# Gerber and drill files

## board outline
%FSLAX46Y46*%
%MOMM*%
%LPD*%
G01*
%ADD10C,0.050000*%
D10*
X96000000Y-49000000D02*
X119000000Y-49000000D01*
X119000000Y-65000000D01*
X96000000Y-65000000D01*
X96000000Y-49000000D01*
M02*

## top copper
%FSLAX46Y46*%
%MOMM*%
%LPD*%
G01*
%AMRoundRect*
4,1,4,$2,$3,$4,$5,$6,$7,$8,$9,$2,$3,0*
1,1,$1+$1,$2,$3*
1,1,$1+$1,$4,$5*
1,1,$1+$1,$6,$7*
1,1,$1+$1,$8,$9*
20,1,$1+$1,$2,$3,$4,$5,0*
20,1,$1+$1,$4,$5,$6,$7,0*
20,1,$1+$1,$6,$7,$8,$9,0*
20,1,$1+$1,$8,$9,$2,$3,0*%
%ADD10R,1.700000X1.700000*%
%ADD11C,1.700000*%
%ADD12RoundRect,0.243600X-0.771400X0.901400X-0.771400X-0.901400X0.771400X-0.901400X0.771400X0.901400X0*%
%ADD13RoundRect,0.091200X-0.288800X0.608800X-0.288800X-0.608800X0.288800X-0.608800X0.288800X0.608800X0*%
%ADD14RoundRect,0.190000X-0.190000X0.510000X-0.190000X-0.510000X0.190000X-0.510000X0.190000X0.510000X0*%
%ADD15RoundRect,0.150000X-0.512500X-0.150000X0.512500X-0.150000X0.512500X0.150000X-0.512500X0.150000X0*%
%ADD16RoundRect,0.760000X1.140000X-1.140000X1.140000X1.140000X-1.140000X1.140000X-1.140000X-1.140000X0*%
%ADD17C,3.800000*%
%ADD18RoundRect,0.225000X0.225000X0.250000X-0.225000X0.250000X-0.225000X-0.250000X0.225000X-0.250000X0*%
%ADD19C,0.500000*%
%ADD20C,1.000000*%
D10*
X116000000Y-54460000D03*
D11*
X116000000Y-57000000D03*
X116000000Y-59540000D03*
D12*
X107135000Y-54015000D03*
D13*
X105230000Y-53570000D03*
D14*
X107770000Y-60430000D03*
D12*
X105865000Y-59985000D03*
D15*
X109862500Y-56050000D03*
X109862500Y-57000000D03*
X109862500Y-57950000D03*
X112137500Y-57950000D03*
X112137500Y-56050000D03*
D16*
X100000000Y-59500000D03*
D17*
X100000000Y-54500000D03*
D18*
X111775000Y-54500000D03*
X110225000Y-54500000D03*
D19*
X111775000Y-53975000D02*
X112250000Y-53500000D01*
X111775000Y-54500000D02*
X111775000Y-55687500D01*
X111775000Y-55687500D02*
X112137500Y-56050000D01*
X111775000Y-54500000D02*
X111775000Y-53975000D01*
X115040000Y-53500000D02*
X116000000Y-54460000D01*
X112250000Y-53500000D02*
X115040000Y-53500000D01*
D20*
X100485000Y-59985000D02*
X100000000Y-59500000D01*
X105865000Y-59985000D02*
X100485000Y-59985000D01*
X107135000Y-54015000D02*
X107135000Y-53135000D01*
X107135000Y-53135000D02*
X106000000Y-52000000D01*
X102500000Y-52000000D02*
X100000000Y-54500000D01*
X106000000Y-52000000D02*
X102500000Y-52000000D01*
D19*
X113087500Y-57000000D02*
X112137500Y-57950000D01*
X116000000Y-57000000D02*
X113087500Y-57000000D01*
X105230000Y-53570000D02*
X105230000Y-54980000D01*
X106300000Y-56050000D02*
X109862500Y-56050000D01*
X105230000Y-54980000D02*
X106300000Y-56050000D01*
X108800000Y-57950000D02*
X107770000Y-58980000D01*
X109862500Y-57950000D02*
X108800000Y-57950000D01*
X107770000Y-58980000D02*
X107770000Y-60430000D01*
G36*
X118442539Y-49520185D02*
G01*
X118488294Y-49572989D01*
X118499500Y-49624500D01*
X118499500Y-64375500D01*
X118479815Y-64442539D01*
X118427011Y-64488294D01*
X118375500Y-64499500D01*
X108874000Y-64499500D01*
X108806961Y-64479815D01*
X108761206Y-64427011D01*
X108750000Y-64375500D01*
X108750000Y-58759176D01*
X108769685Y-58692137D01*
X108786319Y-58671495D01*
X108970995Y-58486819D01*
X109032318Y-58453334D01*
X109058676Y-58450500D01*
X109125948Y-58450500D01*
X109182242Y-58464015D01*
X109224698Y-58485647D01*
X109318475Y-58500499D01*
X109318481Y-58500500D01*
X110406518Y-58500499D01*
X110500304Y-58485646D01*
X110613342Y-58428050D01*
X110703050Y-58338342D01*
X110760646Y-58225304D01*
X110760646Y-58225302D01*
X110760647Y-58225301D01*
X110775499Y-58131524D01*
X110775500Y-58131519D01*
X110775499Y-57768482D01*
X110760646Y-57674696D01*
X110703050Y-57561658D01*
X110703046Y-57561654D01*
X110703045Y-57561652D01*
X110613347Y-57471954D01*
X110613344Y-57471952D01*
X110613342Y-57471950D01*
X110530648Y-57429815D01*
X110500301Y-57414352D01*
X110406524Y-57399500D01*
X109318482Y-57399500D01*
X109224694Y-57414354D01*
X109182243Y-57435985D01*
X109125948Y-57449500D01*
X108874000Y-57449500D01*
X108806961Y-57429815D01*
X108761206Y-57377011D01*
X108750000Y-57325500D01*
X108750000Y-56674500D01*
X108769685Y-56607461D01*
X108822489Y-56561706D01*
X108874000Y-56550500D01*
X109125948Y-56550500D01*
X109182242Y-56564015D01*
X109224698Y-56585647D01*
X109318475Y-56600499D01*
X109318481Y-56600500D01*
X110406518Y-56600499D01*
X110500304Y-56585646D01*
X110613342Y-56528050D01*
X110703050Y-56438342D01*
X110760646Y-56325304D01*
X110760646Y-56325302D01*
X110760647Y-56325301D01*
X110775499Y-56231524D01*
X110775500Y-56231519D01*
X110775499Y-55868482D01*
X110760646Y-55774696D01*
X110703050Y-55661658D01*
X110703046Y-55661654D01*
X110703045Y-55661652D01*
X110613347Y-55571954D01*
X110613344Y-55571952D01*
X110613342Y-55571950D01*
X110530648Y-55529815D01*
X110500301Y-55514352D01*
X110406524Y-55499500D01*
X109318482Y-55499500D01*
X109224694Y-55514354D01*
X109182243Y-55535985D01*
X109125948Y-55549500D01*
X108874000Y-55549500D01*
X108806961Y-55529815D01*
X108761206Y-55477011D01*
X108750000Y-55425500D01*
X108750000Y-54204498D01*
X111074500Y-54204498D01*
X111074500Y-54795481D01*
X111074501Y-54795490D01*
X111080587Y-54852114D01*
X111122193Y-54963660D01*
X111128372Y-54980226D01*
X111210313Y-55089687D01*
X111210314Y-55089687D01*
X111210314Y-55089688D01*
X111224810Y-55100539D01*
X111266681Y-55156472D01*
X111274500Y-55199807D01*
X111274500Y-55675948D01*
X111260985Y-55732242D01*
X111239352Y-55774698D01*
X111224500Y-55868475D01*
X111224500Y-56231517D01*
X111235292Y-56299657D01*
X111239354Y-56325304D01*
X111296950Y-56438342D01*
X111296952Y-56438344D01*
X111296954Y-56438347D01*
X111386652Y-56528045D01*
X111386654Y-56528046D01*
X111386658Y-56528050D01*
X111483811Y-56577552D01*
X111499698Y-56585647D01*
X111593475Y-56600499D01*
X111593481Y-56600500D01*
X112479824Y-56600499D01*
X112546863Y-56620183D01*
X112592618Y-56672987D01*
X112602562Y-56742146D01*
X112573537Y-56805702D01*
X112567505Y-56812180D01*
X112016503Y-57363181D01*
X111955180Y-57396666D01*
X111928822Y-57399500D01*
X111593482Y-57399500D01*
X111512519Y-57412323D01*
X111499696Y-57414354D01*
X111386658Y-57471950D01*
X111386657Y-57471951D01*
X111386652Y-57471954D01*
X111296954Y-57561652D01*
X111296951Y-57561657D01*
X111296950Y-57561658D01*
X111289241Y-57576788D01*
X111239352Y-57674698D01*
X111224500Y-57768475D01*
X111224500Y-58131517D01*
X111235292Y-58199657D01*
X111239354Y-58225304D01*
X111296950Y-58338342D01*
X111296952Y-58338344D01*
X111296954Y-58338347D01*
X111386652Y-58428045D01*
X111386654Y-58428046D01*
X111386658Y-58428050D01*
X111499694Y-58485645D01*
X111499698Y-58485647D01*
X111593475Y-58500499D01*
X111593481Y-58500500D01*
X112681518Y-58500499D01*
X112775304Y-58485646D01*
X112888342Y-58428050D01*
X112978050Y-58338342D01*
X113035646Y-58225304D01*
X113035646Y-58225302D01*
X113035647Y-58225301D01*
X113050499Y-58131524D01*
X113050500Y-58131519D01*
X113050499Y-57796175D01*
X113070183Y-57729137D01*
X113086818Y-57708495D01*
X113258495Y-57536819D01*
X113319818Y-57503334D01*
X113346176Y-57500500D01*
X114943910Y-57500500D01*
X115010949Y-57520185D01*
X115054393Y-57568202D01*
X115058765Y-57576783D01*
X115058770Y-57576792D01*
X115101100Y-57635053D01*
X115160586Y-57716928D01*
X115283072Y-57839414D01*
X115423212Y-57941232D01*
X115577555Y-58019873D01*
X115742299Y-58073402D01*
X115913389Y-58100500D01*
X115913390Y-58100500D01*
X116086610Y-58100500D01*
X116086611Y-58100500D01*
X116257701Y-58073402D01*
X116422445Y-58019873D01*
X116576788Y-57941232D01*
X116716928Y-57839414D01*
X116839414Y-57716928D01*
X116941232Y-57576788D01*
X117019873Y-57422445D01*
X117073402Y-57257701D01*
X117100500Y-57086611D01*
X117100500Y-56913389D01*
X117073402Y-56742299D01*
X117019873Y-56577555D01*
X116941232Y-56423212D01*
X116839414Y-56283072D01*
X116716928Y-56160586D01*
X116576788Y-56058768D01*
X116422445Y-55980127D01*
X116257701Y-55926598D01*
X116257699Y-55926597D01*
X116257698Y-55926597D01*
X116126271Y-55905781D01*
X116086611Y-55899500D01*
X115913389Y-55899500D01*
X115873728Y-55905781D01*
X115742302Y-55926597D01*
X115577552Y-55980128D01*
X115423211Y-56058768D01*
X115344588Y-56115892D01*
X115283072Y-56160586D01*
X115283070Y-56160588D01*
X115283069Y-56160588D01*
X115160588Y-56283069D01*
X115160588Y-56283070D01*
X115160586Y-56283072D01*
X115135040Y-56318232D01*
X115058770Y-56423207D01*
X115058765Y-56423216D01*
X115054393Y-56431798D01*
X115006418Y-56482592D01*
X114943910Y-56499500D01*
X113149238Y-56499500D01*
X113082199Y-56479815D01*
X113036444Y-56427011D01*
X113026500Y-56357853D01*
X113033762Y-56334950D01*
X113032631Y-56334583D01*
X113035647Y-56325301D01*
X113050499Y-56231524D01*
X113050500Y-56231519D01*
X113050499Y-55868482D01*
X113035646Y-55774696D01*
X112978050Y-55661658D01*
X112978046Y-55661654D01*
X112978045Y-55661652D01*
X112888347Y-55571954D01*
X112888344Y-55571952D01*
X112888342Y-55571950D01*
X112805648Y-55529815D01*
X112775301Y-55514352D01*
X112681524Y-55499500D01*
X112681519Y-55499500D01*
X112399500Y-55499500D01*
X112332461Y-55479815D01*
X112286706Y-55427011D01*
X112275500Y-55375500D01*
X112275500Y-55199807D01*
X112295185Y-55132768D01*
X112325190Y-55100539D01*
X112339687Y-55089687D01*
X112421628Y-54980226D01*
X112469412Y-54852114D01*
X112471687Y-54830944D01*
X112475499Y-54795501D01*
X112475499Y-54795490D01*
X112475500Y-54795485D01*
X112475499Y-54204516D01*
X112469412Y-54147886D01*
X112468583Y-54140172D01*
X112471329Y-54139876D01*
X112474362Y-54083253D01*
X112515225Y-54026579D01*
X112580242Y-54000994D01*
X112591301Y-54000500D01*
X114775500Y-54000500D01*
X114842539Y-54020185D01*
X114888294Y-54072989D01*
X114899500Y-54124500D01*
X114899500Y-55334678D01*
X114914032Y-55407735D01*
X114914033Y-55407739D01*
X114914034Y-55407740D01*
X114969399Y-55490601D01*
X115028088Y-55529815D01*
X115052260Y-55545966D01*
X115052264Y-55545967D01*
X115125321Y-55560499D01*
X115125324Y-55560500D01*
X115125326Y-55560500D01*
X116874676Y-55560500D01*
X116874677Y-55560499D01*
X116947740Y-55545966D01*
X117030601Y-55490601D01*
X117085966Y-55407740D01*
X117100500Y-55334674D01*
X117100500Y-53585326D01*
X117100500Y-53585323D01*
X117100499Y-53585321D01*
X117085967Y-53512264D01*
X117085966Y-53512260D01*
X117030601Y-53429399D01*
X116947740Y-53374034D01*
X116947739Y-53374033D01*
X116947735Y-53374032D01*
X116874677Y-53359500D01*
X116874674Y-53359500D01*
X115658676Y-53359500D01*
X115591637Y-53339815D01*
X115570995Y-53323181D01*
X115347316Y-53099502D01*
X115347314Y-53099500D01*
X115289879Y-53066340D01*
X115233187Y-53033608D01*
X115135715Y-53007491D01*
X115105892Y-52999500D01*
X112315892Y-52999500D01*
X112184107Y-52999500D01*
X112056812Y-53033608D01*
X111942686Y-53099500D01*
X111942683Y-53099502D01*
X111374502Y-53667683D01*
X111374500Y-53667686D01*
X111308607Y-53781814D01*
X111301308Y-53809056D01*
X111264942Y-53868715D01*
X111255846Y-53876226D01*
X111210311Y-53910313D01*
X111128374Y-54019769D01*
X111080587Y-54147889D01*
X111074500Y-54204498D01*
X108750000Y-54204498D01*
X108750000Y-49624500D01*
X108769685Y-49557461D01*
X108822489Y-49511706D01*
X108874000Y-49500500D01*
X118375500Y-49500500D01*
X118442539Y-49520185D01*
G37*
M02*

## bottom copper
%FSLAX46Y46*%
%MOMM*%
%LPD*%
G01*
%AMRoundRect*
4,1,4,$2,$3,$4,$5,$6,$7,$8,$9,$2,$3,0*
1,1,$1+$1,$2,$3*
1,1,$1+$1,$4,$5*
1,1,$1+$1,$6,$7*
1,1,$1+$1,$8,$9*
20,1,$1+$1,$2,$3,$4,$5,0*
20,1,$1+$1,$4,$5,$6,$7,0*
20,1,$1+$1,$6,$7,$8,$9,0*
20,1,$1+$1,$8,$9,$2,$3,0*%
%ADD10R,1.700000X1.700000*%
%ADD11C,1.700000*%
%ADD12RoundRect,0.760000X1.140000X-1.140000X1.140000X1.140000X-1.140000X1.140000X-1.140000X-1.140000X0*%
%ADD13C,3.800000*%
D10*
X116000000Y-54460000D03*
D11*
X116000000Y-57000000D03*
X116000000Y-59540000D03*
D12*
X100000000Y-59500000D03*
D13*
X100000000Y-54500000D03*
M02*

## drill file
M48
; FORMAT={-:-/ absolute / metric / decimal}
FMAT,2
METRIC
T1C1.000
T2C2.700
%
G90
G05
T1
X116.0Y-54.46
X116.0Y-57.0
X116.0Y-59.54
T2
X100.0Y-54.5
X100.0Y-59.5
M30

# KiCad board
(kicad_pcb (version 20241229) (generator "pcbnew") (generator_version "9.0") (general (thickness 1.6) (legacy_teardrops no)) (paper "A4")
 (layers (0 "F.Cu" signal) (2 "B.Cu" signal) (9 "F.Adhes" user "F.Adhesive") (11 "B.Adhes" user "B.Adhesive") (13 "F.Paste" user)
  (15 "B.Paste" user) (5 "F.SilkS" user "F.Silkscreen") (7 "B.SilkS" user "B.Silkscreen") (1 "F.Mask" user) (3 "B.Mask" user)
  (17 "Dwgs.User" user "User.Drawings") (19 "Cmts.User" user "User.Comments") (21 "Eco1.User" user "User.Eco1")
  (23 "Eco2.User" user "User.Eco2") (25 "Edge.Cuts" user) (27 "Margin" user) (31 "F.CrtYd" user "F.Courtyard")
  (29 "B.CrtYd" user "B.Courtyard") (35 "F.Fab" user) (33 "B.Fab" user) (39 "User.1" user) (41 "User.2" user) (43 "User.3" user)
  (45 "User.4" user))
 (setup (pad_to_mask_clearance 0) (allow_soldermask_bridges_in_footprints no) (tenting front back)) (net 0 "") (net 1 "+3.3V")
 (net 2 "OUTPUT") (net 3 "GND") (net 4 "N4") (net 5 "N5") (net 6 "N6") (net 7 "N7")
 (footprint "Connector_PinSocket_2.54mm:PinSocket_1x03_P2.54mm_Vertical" (layer "F.Cu") (at 116 54.46)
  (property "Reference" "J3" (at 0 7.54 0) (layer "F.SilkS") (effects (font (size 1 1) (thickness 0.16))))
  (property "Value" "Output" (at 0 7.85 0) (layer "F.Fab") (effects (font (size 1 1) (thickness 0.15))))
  (pad "1" thru_hole rect (at 0 0) (size 1.7 1.7) (drill 1) (layers "*.Cu" "*.Mask") (remove_unused_layers no) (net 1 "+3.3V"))
  (pad "2" thru_hole circle (at 0 2.54) (size 1.7 1.7) (drill 1) (layers "*.Cu" "*.Mask") (remove_unused_layers no) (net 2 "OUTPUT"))
  (pad "3" thru_hole circle (at 0 5.08) (size 1.7 1.7) (drill 1) (layers "*.Cu" "*.Mask") (remove_unused_layers no) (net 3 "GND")))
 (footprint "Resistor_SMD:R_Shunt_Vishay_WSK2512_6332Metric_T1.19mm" (layer "F.Cu") (at 106.5 57 -90)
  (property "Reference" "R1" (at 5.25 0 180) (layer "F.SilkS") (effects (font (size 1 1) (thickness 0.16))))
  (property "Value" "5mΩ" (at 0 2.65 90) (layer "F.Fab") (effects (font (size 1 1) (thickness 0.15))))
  (pad "1" smd roundrect (at -2.985 -0.635 270) (size 2.29 2.03) (layers "F.Cu" "F.Mask" "F.Paste") (roundrect_rratio 0.12) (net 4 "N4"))
  (pad "2" smd roundrect (at -3.43 1.27 270) (size 1.4 0.76) (layers "F.Cu" "F.Mask" "F.Paste") (roundrect_rratio 0.12) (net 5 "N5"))
  (pad "3" smd roundrect (at 3.43 -1.27 270) (size 1.4 0.76) (layers "F.Cu" "F.Mask" "F.Paste") (roundrect_rratio 0.25) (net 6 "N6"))
  (pad "4" smd roundrect (at 2.985 0.635 270) (size 2.29 2.03) (layers "F.Cu" "F.Mask" "F.Paste") (roundrect_rratio 0.12) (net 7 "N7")))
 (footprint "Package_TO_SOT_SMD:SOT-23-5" (layer "F.Cu") (at 111 57)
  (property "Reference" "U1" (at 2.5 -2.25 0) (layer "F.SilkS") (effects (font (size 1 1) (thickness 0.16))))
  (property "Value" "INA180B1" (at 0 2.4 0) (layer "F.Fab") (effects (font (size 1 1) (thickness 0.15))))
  (pad "1" smd roundrect (at -1.1375 -0.95) (size 1.325 0.6) (layers "F.Cu" "F.Mask" "F.Paste") (roundrect_rratio 0.25) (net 5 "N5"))
  (pad "2" smd roundrect (at -1.1375 0) (size 1.325 0.6) (layers "F.Cu" "F.Mask" "F.Paste") (roundrect_rratio 0.25) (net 3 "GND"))
  (pad "3" smd roundrect (at -1.1375 0.95) (size 1.325 0.6) (layers "F.Cu" "F.Mask" "F.Paste") (roundrect_rratio 0.25) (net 6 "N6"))
  (pad "4" smd roundrect (at 1.1375 0.95) (size 1.325 0.6) (layers "F.Cu" "F.Mask" "F.Paste") (roundrect_rratio 0.25) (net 2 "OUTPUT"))
  (pad "5" smd roundrect (at 1.1375 -0.95) (size 1.325 0.6) (layers "F.Cu" "F.Mask" "F.Paste") (roundrect_rratio 0.25) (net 1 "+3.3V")))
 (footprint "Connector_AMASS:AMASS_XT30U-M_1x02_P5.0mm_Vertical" (layer "F.Cu") (at 100 59.5 90)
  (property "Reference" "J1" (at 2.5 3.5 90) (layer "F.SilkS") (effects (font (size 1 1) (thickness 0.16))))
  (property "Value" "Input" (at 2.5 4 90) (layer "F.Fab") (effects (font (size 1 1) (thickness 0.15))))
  (pad "1" thru_hole roundrect (at 0 0 90) (size 3.8 3.8) (drill 2.7) (layers "*.Cu" "*.Mask") (remove_unused_layers no)
   (roundrect_rratio 0.2) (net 7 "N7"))
  (pad "2" thru_hole circle (at 5 0 90) (size 3.8 3.8) (drill 2.7) (layers "*.Cu" "*.Mask") (remove_unused_layers no) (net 4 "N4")))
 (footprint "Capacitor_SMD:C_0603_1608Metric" (layer "F.Cu") (at 111 54.5 180)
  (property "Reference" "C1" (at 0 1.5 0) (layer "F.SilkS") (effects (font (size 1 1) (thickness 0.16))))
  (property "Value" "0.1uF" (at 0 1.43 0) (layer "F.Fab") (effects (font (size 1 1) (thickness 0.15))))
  (pad "1" smd roundrect (at -0.775 0 180) (size 0.9 0.95) (layers "F.Cu" "F.Mask" "F.Paste") (roundrect_rratio 0.25) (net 1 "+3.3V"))
  (pad "2" smd roundrect (at 0.775 0 180) (size 0.9 0.95) (layers "F.Cu" "F.Mask" "F.Paste") (roundrect_rratio 0.25) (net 3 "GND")))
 (gr_rect (start 96 49) (end 119 65) (stroke (width 0.05) (type default)) (fill no) (layer "Edge.Cuts"))
 (segment (start 111.775 53.975) (end 112.25 53.5) (width 0.5) (layer "F.Cu") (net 1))
 (segment (start 111.775 54.5) (end 111.775 55.6875) (width 0.5) (layer "F.Cu") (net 1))
 (segment (start 111.775 55.6875) (end 112.1375 56.05) (width 0.5) (layer "F.Cu") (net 1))
 (segment (start 111.775 54.5) (end 111.775 53.975) (width 0.5) (layer "F.Cu") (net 1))
 (segment (start 115.04 53.5) (end 116 54.46) (width 0.5) (layer "F.Cu") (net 1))
 (segment (start 112.25 53.5) (end 115.04 53.5) (width 0.5) (layer "F.Cu") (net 1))
 (segment (start 100.485 59.985) (end 100 59.5) (width 1) (layer "F.Cu") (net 7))
 (segment (start 105.865 59.985) (end 100.485 59.985) (width 1) (layer "F.Cu") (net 7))
 (segment (start 107.135 54.015) (end 107.135 53.135) (width 1) (layer "F.Cu") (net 4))
 (segment (start 107.135 53.135) (end 106 52) (width 1) (layer "F.Cu") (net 4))
 (segment (start 102.5 52) (end 100 54.5) (width 1) (layer "F.Cu") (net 4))
 (segment (start 106 52) (end 102.5 52) (width 1) (layer "F.Cu") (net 4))
 (segment (start 113.0875 57) (end 112.1375 57.95) (width 0.5) (layer "F.Cu") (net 2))
 (segment (start 116 57) (end 113.0875 57) (width 0.5) (layer "F.Cu") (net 2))
 (segment (start 105.23 53.57) (end 105.23 54.98) (width 0.5) (layer "F.Cu") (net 5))
 (segment (start 106.3 56.05) (end 109.8625 56.05) (width 0.5) (layer "F.Cu") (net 5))
 (segment (start 105.23 54.98) (end 106.3 56.05) (width 0.5) (layer "F.Cu") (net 5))
 (segment (start 108.8 57.95) (end 107.77 58.98) (width 0.5) (layer "F.Cu") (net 6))
 (segment (start 109.8625 57.95) (end 108.8 57.95) (width 0.5) (layer "F.Cu") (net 6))
 (segment (start 107.77 58.98) (end 107.77 60.43) (width 0.5) (layer "F.Cu") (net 6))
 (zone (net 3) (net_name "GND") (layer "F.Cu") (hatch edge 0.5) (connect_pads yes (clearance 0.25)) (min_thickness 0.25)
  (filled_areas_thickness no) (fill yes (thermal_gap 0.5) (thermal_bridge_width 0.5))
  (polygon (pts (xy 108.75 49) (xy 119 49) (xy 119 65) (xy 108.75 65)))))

